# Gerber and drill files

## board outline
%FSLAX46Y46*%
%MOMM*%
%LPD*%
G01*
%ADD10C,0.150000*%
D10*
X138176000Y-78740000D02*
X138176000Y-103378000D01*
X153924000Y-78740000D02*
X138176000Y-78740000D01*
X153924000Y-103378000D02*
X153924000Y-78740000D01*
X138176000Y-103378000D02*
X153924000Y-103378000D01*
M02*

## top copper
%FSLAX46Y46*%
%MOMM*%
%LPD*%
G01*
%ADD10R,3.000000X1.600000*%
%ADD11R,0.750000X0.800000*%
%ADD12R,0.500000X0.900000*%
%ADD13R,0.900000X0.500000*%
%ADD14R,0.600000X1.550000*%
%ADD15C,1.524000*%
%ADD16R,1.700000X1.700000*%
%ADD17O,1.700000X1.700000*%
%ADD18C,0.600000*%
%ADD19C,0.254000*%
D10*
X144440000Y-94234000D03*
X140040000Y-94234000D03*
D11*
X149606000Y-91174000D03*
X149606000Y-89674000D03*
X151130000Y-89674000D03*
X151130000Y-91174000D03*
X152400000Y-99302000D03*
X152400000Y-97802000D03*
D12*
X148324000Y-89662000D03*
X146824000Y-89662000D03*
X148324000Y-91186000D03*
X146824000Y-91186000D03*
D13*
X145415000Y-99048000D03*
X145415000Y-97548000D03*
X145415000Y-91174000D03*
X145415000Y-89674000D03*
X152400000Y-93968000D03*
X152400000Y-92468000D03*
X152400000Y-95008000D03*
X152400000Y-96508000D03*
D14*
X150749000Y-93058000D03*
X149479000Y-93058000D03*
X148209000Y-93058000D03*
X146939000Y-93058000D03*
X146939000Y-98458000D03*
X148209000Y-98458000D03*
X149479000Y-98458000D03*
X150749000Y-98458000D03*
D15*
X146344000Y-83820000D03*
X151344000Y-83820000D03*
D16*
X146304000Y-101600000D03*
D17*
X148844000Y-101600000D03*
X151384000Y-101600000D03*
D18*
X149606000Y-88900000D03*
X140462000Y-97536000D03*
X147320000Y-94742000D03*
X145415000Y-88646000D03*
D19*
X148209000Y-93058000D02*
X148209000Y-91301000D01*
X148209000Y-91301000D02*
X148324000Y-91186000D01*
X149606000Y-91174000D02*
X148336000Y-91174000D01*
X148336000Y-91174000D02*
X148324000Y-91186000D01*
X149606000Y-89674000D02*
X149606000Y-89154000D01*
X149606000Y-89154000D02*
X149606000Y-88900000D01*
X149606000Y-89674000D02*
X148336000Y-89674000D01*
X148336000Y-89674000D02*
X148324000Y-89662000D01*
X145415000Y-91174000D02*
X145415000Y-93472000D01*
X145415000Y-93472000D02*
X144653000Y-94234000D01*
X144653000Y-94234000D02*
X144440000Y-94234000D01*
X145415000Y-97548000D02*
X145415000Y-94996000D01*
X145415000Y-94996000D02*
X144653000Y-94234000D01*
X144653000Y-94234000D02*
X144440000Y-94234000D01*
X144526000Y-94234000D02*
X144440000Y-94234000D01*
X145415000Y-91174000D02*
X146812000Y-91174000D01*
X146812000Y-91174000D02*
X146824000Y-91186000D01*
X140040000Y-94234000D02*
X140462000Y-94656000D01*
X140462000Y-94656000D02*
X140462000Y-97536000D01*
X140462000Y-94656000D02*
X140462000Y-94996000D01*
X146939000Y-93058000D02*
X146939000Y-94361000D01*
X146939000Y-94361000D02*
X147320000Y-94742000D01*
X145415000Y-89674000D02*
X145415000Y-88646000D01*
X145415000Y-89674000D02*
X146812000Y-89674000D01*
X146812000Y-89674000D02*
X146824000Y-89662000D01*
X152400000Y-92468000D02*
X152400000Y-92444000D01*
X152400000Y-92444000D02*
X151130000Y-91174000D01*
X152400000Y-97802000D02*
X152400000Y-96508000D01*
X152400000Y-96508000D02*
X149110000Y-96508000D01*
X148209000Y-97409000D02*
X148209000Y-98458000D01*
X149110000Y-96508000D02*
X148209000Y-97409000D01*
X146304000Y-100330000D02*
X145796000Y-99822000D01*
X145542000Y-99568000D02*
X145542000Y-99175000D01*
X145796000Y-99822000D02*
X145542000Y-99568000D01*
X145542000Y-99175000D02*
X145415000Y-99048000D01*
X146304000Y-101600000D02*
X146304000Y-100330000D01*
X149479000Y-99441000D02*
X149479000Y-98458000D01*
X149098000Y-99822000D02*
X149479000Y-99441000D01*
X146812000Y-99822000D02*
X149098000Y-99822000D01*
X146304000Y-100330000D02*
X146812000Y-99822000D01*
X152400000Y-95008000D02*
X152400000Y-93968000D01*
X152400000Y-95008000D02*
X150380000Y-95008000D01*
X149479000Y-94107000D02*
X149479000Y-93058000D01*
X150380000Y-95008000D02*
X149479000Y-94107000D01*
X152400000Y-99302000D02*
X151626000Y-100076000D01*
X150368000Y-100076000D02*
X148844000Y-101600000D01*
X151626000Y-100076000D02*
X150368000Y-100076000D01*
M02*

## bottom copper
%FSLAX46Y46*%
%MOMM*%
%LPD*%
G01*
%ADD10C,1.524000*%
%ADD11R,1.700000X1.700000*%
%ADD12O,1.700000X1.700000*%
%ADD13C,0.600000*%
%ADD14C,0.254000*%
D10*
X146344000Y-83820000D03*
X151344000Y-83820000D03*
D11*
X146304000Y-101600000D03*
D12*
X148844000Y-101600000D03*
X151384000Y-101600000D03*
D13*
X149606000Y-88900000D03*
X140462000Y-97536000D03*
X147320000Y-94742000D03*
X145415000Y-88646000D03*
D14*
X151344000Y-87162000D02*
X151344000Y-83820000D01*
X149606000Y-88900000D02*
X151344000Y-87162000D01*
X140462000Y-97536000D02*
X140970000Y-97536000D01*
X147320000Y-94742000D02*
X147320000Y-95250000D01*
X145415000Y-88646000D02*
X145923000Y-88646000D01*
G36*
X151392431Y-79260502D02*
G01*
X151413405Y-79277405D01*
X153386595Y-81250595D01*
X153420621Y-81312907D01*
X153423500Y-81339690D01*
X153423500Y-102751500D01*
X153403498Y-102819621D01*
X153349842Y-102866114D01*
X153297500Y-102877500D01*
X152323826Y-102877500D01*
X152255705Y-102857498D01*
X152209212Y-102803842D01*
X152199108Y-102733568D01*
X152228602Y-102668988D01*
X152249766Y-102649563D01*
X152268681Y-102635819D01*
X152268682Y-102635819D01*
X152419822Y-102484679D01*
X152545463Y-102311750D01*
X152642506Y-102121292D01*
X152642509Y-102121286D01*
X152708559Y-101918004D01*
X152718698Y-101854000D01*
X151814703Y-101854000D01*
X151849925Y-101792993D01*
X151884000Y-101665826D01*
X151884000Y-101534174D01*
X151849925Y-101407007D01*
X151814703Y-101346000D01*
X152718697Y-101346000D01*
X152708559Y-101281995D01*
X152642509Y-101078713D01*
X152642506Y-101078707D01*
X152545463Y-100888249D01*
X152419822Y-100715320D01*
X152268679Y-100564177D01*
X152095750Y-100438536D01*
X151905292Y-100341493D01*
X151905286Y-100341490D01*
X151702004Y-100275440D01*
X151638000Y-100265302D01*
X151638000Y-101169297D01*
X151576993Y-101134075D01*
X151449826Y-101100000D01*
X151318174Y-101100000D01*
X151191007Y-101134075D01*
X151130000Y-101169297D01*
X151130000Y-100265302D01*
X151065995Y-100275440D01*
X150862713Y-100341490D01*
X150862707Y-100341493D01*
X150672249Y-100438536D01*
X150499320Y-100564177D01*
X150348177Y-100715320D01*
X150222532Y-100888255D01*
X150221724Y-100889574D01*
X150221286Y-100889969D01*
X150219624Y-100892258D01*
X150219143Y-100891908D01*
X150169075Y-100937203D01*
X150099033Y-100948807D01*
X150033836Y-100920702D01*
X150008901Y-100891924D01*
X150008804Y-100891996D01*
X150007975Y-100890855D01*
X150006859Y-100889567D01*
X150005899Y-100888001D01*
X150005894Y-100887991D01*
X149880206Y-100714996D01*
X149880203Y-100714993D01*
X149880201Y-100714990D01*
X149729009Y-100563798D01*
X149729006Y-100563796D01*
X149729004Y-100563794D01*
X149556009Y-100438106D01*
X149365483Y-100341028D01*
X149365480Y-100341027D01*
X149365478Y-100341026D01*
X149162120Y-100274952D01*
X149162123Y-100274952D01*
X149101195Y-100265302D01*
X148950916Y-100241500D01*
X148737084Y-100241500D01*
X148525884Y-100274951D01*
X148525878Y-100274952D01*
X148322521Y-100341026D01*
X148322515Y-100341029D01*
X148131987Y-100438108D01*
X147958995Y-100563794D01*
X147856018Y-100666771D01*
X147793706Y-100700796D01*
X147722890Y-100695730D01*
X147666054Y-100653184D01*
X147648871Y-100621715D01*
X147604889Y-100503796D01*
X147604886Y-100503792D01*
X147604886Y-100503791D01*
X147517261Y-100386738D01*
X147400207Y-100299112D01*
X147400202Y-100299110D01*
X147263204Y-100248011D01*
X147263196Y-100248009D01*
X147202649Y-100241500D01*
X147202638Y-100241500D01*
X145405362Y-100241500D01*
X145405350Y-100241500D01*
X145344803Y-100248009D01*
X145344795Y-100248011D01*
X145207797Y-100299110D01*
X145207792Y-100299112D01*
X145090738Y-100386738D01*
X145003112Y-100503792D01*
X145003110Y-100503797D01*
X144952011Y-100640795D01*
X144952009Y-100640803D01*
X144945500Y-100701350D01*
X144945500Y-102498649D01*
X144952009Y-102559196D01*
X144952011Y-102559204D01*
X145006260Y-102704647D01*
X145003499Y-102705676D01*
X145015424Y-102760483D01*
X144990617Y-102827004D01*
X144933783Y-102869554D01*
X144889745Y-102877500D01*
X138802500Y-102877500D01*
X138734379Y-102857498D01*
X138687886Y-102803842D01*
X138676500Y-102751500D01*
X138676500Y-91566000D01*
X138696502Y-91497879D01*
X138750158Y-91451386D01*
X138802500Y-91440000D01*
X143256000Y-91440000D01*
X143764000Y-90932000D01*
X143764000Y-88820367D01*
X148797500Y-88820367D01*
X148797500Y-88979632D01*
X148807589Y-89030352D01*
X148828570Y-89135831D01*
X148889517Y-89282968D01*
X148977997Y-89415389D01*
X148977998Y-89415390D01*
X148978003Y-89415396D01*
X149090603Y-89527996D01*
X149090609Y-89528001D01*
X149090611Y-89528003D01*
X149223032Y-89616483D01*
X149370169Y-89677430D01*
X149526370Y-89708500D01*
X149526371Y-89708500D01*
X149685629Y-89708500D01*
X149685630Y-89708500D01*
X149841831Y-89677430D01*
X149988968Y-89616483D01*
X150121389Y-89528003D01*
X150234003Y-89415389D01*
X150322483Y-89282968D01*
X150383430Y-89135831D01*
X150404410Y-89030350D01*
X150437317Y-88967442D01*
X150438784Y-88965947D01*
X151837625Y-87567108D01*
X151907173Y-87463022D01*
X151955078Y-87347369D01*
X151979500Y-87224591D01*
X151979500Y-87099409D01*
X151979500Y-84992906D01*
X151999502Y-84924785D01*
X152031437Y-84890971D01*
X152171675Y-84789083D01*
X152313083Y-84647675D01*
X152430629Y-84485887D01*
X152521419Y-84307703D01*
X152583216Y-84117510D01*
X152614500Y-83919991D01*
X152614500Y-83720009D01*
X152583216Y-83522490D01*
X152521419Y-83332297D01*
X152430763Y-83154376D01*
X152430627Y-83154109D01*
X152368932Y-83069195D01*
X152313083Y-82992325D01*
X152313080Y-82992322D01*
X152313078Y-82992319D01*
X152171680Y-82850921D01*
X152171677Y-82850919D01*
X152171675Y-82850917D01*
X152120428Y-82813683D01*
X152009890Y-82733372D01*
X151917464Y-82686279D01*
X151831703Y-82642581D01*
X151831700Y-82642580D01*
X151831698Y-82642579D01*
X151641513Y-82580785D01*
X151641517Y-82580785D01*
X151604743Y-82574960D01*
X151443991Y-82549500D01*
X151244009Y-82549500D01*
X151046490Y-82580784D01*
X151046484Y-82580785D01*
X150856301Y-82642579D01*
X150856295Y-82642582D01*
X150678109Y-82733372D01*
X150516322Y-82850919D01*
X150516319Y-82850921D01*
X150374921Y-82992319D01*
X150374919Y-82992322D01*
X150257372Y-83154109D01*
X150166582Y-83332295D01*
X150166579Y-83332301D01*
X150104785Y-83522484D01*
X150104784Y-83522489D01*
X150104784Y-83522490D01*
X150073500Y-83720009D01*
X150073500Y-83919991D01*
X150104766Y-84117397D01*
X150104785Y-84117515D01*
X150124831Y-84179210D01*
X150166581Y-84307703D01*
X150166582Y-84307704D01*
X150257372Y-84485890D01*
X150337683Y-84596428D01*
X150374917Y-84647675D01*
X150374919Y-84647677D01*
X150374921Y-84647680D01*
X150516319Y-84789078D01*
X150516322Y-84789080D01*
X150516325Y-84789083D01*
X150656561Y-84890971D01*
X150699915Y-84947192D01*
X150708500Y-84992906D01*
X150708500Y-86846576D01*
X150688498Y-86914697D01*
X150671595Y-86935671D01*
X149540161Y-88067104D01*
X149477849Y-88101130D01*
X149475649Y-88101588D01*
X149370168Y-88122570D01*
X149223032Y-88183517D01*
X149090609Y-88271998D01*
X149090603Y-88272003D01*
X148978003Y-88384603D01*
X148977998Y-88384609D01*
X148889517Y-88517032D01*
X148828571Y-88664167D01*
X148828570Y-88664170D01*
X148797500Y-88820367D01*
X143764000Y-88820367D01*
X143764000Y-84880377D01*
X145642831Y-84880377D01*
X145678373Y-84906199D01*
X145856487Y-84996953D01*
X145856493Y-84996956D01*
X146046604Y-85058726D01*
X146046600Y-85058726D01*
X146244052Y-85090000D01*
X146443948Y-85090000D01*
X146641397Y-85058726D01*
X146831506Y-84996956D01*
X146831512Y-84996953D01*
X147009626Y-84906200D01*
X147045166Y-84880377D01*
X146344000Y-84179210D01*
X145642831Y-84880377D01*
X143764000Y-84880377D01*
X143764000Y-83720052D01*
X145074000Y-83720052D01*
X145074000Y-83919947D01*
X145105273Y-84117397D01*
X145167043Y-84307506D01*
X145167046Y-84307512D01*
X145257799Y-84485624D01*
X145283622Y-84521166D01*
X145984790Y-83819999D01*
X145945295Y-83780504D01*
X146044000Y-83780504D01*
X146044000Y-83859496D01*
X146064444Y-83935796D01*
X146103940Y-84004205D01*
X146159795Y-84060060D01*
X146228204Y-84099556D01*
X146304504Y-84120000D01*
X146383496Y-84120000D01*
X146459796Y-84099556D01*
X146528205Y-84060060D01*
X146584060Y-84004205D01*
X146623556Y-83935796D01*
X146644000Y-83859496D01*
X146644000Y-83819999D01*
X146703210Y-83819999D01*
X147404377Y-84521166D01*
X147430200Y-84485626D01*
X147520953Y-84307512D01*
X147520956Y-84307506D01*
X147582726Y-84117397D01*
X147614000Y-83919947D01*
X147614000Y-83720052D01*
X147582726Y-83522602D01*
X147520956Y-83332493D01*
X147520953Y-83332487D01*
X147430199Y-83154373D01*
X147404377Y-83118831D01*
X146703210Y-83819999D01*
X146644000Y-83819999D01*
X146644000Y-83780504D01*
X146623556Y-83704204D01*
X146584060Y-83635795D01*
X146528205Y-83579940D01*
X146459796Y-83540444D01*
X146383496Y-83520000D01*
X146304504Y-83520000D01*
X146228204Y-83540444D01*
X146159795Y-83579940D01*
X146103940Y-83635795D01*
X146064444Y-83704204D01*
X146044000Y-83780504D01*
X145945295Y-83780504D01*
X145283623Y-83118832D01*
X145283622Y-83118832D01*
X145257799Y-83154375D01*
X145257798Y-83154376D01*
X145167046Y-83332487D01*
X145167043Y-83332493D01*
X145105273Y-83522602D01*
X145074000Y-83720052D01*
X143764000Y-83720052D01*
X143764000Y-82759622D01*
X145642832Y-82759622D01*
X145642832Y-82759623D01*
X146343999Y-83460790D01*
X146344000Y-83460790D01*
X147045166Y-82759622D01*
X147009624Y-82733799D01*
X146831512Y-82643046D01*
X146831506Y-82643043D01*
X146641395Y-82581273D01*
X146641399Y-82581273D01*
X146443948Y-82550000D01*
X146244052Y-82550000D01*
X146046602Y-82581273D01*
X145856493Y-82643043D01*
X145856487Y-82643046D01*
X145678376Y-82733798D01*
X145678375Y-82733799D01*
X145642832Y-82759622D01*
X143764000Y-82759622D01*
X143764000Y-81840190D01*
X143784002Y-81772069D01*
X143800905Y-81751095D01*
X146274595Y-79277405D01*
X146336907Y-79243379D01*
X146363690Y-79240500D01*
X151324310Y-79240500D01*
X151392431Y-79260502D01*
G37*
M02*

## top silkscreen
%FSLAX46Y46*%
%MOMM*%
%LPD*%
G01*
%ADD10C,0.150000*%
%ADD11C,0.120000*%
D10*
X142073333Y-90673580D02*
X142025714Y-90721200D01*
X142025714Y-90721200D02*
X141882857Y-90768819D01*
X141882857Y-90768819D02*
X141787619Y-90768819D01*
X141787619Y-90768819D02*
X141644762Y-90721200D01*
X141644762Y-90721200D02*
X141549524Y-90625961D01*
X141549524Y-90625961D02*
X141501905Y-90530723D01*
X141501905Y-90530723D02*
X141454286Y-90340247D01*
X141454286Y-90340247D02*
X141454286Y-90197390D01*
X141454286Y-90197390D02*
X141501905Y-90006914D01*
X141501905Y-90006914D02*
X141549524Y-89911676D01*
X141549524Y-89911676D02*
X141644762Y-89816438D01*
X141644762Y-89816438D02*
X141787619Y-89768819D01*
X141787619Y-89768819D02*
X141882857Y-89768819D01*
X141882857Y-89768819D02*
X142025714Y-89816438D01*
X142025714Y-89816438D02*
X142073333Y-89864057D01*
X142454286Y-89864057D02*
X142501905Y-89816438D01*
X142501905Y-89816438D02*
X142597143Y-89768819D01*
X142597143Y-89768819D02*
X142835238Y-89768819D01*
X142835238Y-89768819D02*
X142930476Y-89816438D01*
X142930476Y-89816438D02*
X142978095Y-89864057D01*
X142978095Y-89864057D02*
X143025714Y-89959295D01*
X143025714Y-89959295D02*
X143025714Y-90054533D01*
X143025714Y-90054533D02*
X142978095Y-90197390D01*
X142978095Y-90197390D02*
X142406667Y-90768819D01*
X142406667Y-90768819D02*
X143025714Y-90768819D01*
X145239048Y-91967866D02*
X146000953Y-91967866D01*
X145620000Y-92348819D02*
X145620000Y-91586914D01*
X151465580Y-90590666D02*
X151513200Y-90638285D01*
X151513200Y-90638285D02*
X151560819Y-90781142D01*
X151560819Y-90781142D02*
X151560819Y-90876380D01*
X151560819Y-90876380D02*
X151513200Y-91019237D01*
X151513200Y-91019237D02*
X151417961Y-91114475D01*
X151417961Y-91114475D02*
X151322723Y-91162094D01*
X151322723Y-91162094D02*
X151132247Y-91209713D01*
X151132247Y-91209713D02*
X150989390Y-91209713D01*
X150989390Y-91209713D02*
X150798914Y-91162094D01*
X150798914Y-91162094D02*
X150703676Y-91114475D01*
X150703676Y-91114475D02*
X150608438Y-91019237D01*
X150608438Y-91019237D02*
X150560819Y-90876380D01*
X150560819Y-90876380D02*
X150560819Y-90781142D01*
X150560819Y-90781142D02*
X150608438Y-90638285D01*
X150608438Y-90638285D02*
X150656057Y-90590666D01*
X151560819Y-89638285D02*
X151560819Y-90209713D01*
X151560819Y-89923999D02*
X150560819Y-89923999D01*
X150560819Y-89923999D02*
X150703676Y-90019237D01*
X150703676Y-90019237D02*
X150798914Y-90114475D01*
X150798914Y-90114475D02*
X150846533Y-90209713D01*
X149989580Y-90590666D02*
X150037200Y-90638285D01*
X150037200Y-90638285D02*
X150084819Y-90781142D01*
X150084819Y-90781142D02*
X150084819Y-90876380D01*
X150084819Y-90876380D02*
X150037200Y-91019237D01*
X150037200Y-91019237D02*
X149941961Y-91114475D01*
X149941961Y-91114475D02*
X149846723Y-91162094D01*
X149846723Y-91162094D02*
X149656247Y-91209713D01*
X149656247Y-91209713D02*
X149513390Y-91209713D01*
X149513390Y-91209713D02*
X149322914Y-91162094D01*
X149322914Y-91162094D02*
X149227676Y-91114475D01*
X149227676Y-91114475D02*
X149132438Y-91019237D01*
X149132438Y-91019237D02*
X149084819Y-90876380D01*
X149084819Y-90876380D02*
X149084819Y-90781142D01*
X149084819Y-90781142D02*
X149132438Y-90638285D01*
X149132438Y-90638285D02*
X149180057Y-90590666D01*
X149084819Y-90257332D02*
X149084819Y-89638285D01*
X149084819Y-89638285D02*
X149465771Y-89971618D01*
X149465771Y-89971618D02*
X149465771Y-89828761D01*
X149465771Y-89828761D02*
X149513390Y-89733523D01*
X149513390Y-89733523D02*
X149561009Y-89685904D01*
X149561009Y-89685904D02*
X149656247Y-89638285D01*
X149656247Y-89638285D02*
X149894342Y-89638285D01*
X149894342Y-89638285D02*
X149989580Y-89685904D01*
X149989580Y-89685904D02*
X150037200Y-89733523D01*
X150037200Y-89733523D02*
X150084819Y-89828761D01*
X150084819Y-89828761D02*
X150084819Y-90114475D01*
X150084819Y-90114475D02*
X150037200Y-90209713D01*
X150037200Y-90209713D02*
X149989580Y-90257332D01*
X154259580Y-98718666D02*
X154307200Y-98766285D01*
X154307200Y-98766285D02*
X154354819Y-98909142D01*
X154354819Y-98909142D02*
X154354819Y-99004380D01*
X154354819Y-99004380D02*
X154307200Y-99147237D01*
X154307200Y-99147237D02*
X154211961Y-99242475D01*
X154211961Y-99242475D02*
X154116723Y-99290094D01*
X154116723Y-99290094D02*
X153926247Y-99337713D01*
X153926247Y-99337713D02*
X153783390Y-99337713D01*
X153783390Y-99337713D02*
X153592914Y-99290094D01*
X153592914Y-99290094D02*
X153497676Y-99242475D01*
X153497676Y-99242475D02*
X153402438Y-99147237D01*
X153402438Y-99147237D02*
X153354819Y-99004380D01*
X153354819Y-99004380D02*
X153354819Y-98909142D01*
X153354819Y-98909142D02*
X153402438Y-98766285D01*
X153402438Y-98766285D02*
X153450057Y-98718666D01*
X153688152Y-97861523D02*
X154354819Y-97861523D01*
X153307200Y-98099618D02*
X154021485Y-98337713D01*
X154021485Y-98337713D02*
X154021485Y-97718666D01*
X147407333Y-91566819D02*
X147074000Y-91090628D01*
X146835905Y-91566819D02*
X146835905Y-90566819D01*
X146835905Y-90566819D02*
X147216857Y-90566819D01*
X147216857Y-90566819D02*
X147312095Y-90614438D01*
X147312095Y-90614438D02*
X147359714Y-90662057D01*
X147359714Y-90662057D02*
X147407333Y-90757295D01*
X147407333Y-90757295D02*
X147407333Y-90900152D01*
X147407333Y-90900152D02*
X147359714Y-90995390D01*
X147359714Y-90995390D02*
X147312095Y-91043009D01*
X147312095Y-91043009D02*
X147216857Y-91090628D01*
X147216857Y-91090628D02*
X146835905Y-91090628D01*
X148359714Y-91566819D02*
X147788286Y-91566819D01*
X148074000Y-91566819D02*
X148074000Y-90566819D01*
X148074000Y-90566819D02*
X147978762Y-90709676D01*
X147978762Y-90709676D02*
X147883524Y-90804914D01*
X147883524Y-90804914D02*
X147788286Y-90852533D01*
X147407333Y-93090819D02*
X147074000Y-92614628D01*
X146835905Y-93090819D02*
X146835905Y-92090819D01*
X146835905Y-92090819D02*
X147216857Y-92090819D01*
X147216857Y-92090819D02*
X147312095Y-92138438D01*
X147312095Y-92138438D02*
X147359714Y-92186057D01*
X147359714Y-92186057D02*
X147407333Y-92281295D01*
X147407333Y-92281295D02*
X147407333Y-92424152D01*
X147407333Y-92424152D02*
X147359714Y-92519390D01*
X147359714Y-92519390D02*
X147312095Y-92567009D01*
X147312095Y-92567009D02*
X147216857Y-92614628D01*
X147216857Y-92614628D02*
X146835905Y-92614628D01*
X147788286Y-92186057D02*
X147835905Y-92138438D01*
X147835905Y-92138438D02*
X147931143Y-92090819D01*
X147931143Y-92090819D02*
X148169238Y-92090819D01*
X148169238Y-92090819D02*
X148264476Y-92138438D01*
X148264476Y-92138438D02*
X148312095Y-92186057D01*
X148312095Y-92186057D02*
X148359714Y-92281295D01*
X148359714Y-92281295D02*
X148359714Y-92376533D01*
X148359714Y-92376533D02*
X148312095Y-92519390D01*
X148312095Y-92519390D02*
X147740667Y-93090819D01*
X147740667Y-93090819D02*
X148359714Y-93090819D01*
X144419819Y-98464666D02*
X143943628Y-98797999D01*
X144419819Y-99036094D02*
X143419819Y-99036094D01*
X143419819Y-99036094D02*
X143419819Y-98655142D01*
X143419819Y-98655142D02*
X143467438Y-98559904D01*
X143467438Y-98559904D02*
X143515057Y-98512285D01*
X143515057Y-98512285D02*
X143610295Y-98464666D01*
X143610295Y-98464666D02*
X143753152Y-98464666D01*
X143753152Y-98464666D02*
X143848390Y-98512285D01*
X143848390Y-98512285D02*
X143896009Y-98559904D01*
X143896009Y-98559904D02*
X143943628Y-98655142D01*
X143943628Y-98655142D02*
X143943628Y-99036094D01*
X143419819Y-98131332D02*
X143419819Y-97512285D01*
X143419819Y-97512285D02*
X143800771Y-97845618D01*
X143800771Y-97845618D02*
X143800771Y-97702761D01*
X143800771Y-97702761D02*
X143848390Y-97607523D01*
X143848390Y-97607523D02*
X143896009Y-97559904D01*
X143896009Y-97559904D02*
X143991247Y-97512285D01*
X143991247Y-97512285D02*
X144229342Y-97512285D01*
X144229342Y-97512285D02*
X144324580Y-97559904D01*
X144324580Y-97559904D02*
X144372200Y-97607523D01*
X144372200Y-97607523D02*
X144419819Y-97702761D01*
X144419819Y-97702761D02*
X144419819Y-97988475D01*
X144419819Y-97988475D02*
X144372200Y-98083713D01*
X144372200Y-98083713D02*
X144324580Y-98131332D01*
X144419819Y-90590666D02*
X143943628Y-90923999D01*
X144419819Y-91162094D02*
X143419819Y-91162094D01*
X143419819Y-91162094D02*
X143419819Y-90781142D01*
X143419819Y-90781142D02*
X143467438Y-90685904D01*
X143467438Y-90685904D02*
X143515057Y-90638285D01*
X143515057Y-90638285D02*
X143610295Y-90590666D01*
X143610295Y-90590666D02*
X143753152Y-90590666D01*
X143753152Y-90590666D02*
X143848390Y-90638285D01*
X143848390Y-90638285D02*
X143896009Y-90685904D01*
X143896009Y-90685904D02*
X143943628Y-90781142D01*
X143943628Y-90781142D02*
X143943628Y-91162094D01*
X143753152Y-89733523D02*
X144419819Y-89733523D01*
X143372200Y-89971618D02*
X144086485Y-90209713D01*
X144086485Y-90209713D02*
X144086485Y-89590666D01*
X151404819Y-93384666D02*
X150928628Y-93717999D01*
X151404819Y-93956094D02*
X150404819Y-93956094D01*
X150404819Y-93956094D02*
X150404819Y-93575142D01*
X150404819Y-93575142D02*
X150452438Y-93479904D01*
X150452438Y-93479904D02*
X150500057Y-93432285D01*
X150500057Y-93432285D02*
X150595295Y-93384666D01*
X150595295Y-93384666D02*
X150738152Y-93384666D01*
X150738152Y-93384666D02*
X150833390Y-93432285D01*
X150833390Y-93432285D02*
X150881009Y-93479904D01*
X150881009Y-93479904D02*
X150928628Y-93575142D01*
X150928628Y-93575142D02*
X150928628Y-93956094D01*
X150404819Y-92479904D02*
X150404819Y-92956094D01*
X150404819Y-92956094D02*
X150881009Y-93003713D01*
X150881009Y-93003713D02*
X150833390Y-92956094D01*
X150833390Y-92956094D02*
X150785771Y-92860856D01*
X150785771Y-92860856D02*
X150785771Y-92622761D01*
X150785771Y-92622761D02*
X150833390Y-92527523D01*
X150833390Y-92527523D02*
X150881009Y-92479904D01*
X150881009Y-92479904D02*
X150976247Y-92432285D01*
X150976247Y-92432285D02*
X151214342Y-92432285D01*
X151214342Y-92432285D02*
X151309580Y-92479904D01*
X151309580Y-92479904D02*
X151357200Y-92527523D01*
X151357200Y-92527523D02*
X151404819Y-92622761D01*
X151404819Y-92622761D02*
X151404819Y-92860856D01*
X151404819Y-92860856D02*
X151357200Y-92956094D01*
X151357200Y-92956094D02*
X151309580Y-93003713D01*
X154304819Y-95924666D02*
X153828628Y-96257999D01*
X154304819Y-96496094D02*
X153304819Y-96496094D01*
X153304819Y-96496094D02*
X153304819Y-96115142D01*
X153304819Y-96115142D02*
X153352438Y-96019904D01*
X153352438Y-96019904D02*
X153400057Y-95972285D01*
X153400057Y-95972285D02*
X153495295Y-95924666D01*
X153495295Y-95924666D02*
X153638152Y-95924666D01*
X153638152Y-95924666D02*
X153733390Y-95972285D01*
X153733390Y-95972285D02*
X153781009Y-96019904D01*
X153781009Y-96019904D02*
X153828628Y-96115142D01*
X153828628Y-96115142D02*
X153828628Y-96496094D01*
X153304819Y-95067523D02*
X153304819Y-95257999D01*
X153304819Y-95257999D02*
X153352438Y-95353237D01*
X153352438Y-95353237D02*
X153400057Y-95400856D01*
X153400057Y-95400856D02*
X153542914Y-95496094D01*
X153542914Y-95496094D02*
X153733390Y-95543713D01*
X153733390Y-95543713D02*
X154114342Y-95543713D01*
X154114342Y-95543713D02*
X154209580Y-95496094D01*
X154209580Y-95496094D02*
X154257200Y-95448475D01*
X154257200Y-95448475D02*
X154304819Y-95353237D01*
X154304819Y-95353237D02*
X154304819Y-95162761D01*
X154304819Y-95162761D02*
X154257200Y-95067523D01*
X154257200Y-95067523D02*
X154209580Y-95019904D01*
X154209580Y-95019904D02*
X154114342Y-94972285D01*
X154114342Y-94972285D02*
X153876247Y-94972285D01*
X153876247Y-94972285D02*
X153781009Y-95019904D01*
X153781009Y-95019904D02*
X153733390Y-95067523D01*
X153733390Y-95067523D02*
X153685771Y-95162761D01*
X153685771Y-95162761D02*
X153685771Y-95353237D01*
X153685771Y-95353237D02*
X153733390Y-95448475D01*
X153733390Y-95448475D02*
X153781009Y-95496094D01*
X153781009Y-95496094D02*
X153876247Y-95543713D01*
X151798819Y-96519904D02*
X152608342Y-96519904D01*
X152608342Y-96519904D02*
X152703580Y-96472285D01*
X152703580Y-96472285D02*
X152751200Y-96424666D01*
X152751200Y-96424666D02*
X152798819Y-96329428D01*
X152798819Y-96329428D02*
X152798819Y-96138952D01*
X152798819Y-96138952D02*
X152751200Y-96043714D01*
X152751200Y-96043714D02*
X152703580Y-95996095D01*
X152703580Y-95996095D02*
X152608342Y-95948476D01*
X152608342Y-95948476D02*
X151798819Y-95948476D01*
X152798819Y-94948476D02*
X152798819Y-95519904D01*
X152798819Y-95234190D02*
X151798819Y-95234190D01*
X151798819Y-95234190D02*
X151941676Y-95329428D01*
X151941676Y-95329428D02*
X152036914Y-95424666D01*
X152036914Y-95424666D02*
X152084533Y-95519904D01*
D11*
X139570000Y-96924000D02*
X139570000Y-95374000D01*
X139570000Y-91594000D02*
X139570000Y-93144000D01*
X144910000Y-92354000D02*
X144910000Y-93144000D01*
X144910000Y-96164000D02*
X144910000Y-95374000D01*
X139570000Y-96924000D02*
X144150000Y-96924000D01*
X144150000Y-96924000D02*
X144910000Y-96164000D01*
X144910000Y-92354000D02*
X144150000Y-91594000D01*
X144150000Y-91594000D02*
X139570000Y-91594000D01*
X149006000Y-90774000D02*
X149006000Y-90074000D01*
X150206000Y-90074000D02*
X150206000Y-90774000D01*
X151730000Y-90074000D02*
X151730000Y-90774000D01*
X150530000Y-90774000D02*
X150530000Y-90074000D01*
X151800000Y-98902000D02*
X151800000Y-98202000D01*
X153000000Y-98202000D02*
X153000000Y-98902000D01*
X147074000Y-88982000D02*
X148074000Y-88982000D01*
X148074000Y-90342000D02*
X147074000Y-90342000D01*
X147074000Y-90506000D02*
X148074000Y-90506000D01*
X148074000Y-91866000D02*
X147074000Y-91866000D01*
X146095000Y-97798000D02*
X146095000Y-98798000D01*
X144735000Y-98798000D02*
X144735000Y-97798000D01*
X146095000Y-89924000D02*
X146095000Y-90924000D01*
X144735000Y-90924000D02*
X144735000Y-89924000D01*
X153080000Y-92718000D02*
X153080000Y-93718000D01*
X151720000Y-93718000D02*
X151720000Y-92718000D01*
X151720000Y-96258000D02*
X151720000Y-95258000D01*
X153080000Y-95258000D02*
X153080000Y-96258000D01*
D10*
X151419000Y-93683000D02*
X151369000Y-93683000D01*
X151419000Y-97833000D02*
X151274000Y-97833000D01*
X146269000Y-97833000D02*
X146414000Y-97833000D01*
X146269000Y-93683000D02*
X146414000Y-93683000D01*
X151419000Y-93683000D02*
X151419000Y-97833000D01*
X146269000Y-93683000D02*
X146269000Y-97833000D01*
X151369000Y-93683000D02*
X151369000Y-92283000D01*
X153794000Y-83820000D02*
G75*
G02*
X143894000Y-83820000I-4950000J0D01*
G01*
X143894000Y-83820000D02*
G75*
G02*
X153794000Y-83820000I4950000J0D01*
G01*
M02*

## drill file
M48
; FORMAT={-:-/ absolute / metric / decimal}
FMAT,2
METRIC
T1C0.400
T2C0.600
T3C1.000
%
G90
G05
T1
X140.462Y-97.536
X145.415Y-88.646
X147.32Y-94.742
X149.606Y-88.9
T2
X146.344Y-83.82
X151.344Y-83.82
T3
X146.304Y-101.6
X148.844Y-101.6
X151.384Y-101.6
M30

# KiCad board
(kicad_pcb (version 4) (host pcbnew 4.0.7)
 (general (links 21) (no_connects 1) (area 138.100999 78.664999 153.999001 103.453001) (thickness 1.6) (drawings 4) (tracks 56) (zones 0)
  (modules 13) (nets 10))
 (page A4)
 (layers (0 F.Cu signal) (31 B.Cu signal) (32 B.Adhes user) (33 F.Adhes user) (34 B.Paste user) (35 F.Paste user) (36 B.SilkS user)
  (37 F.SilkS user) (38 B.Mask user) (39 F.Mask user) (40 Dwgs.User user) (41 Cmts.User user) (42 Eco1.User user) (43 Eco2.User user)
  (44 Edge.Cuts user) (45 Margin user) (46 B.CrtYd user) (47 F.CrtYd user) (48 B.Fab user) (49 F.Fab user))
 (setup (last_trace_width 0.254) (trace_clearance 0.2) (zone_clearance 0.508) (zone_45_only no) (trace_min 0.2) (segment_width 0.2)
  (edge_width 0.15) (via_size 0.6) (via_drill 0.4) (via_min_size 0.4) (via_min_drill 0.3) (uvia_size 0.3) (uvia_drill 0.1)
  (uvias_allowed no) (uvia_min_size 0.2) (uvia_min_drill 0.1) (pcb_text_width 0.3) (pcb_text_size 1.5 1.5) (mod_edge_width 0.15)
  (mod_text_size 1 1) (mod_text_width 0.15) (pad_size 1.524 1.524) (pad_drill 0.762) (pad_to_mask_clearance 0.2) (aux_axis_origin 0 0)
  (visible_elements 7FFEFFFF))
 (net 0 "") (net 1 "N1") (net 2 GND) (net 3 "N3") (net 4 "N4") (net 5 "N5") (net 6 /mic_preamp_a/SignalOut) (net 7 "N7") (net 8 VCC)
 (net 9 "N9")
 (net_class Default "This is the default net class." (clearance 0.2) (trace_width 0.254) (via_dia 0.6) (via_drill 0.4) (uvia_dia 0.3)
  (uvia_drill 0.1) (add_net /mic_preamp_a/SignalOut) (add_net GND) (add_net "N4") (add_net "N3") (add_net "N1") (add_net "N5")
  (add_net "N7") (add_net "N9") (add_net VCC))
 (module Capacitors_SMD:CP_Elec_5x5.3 (layer F.Cu) (at 142.24 94.234 180)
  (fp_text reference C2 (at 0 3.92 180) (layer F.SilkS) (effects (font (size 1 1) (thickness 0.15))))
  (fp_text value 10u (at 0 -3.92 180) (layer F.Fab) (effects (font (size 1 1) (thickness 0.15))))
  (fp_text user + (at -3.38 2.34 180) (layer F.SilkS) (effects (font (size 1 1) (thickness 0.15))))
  (fp_line (start 2.67 -2.69) (end 2.67 -1.14) (layer F.SilkS) (width 0.12))
  (fp_line (start 2.67 2.64) (end 2.67 1.09) (layer F.SilkS) (width 0.12))
  (fp_line (start -2.67 1.88) (end -2.67 1.09) (layer F.SilkS) (width 0.12))
  (fp_line (start -2.67 -1.93) (end -2.67 -1.14) (layer F.SilkS) (width 0.12))
  (fp_line (start 2.67 -2.69) (end -1.91 -2.69) (layer F.SilkS) (width 0.12))
  (fp_line (start -1.91 -2.69) (end -2.67 -1.93) (layer F.SilkS) (width 0.12))
  (fp_line (start -2.67 1.88) (end -1.91 2.64) (layer F.SilkS) (width 0.12))
  (fp_line (start -1.91 2.64) (end 2.67 2.64) (layer F.SilkS) (width 0.12))
  (pad 1 smd rect (at -2.2 0) (size 3 1.6) (layers F.Cu F.Paste F.Mask) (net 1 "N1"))
  (pad 2 smd rect (at 2.2 0) (size 3 1.6) (layers F.Cu F.Paste F.Mask) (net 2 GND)))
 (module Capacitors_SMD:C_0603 (layer F.Cu) (at 149.606 90.424 270)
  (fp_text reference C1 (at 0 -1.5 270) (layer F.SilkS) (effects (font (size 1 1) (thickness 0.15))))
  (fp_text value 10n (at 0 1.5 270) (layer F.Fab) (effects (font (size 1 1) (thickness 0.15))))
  (fp_line (start 0.35 0.6) (end -0.35 0.6) (layer F.SilkS) (width 0.12))
  (fp_line (start -0.35 -0.6) (end 0.35 -0.6) (layer F.SilkS) (width 0.12))
  (pad 2 smd rect (at 0.75 0 270) (size 0.8 0.75) (layers F.Cu F.Paste F.Mask) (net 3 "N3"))
  (pad 1 smd rect (at -0.75 0 270) (size 0.8 0.75) (layers F.Cu F.Paste F.Mask) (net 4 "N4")))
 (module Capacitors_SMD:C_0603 (layer F.Cu) (at 151.13 90.424 90)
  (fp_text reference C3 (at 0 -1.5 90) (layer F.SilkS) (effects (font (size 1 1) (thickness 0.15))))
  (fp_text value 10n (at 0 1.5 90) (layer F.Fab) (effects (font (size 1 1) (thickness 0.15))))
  (fp_line (start 0.35 0.6) (end -0.35 0.6) (layer F.SilkS) (width 0.12))
  (fp_line (start -0.35 -0.6) (end 0.35 -0.6) (layer F.SilkS) (width 0.12))
  (pad 2 smd rect (at 0.75 0 90) (size 0.8 0.75) (layers F.Cu F.Paste F.Mask) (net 2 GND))
  (pad 1 smd rect (at -0.75 0 90) (size 0.8 0.75) (layers F.Cu F.Paste F.Mask) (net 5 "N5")))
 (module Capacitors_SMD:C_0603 (layer F.Cu) (at 152.4 98.552 270)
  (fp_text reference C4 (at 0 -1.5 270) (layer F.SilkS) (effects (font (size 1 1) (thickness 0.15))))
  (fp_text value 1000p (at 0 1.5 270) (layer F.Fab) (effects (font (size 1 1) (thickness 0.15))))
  (fp_line (start 0.35 0.6) (end -0.35 0.6) (layer F.SilkS) (width 0.12))
  (fp_line (start -0.35 -0.6) (end 0.35 -0.6) (layer F.SilkS) (width 0.12))
  (pad 2 smd rect (at 0.75 0 270) (size 0.8 0.75) (layers F.Cu F.Paste F.Mask) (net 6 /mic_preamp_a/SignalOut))
  (pad 1 smd rect (at -0.75 0 270) (size 0.8 0.75) (layers F.Cu F.Paste F.Mask) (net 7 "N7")))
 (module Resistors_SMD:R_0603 (layer F.Cu) (at 147.574 89.662 180)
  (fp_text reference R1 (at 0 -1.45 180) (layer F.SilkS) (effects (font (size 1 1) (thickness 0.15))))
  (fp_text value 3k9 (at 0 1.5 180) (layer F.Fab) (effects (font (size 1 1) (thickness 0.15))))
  (fp_line (start 0.5 0.68) (end -0.5 0.68) (layer F.SilkS) (width 0.12))
  (fp_line (start -0.5 -0.68) (end 0.5 -0.68) (layer F.SilkS) (width 0.12))
  (pad 1 smd rect (at -0.75 0 180) (size 0.5 0.9) (layers F.Cu F.Paste F.Mask) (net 4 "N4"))
  (pad 2 smd rect (at 0.75 0 180) (size 0.5 0.9) (layers F.Cu F.Paste F.Mask) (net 2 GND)))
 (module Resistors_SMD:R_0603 (layer F.Cu) (at 147.574 91.186 180)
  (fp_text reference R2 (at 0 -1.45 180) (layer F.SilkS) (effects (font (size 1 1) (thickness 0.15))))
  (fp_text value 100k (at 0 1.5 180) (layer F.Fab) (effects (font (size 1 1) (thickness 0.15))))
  (fp_line (start 0.5 0.68) (end -0.5 0.68) (layer F.SilkS) (width 0.12))
  (fp_line (start -0.5 -0.68) (end 0.5 -0.68) (layer F.SilkS) (width 0.12))
  (pad 1 smd rect (at -0.75 0 180) (size 0.5 0.9) (layers F.Cu F.Paste F.Mask) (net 3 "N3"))
  (pad 2 smd rect (at 0.75 0 180) (size 0.5 0.9) (layers F.Cu F.Paste F.Mask) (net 1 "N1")))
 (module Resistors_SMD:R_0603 (layer F.Cu) (at 145.415 98.298 90)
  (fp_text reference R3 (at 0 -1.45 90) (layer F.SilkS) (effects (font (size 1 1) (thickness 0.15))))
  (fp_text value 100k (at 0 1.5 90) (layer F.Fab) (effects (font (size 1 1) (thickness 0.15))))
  (fp_line (start 0.5 0.68) (end -0.5 0.68) (layer F.SilkS) (width 0.12))
  (fp_line (start -0.5 -0.68) (end 0.5 -0.68) (layer F.SilkS) (width 0.12))
  (pad 1 smd rect (at -0.75 0 90) (size 0.5 0.9) (layers F.Cu F.Paste F.Mask) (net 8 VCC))
  (pad 2 smd rect (at 0.75 0 90) (size 0.5 0.9) (layers F.Cu F.Paste F.Mask) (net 1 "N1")))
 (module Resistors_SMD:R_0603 (layer F.Cu) (at 145.415 90.424 90)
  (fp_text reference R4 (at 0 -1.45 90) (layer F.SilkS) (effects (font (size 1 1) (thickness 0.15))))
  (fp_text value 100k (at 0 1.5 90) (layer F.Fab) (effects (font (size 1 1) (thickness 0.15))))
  (fp_line (start 0.5 0.68) (end -0.5 0.68) (layer F.SilkS) (width 0.12))
  (fp_line (start -0.5 -0.68) (end 0.5 -0.68) (layer F.SilkS) (width 0.12))
  (pad 1 smd rect (at -0.75 0 90) (size 0.5 0.9) (layers F.Cu F.Paste F.Mask) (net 1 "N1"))
  (pad 2 smd rect (at 0.75 0 90) (size 0.5 0.9) (layers F.Cu F.Paste F.Mask) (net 2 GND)))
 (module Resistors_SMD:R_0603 (layer F.Cu) (at 152.4 93.218 90)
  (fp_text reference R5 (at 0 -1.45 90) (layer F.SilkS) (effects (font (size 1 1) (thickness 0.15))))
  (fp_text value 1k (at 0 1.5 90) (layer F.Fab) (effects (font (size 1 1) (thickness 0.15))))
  (fp_line (start 0.5 0.68) (end -0.5 0.68) (layer F.SilkS) (width 0.12))
  (fp_line (start -0.5 -0.68) (end 0.5 -0.68) (layer F.SilkS) (width 0.12))
  (pad 1 smd rect (at -0.75 0 90) (size 0.5 0.9) (layers F.Cu F.Paste F.Mask) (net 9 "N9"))
  (pad 2 smd rect (at 0.75 0 90) (size 0.5 0.9) (layers F.Cu F.Paste F.Mask) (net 5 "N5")))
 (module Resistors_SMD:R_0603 (layer F.Cu) (at 152.4 95.758 270)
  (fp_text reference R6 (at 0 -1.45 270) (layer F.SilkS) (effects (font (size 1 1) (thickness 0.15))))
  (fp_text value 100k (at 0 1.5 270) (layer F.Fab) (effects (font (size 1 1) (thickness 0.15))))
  (fp_line (start 0.5 0.68) (end -0.5 0.68) (layer F.SilkS) (width 0.12))
  (fp_line (start -0.5 -0.68) (end 0.5 -0.68) (layer F.SilkS) (width 0.12))
  (pad 1 smd rect (at -0.75 0 270) (size 0.5 0.9) (layers F.Cu F.Paste F.Mask) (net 9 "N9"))
  (pad 2 smd rect (at 0.75 0 270) (size 0.5 0.9) (layers F.Cu F.Paste F.Mask) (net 7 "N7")))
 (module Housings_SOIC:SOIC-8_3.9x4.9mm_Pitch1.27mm (layer F.Cu) (at 148.844 95.758 270)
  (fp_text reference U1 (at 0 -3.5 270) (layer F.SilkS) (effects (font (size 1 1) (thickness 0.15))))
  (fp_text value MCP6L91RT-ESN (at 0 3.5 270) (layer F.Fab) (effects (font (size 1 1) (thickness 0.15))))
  (fp_line (start -2.075 -2.575) (end -2.075 -2.525) (layer F.SilkS) (width 0.15))
  (fp_line (start 2.075 -2.575) (end 2.075 -2.43) (layer F.SilkS) (width 0.15))
  (fp_line (start 2.075 2.575) (end 2.075 2.43) (layer F.SilkS) (width 0.15))
  (fp_line (start -2.075 2.575) (end -2.075 2.43) (layer F.SilkS) (width 0.15))
  (fp_line (start -2.075 -2.575) (end 2.075 -2.575) (layer F.SilkS) (width 0.15))
  (fp_line (start -2.075 2.575) (end 2.075 2.575) (layer F.SilkS) (width 0.15))
  (fp_line (start -2.075 -2.525) (end -3.475 -2.525) (layer F.SilkS) (width 0.15))
  (pad 1 smd rect (at -2.7 -1.905 270) (size 1.55 0.6) (layers F.Cu F.Paste F.Mask))
  (pad 2 smd rect (at -2.7 -0.635 270) (size 1.55 0.6) (layers F.Cu F.Paste F.Mask) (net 9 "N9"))
  (pad 3 smd rect (at -2.7 0.635 270) (size 1.55 0.6) (layers F.Cu F.Paste F.Mask) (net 3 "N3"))
  (pad 4 smd rect (at -2.7 1.905 270) (size 1.55 0.6) (layers F.Cu F.Paste F.Mask) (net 2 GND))
  (pad 5 smd rect (at 2.7 1.905 270) (size 1.55 0.6) (layers F.Cu F.Paste F.Mask))
  (pad 6 smd rect (at 2.7 0.635 270) (size 1.55 0.6) (layers F.Cu F.Paste F.Mask) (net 7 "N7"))
  (pad 7 smd rect (at 2.7 -0.635 270) (size 1.55 0.6) (layers F.Cu F.Paste F.Mask) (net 8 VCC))
  (pad 8 smd rect (at 2.7 -1.905 270) (size 1.55 0.6) (layers F.Cu F.Paste F.Mask)))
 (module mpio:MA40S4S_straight (layer F.Cu) (at 148.844 83.82)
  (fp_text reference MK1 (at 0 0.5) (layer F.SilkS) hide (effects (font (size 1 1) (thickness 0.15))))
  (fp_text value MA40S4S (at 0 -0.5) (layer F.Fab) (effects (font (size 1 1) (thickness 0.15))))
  (fp_circle (center 0 0) (end 4.95 0) (layer F.SilkS) (width 0.15))
  (pad 1 thru_hole circle (at -2.5 0) (size 1.524 1.524) (drill 0.6) (layers *.Cu *.Mask) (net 2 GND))
  (pad 2 thru_hole circle (at 2.5 0) (size 1.524 1.524) (drill 0.6) (layers *.Cu *.Mask) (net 4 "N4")))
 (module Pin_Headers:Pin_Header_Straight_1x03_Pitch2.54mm (layer B.Cu) (at 146.304 101.6 270)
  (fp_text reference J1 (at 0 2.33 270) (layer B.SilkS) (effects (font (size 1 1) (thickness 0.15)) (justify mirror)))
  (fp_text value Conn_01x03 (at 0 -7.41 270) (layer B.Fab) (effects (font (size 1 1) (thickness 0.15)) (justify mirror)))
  (pad 1 thru_hole rect (at 0 0 270) (size 1.7 1.7) (drill 1) (layers *.Cu *.Mask) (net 8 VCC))
  (pad 2 thru_hole oval (at 0 -2.54 270) (size 1.7 1.7) (drill 1) (layers *.Cu *.Mask) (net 6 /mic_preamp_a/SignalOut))
  (pad 3 thru_hole oval (at 0 -5.08 270) (size 1.7 1.7) (drill 1) (layers *.Cu *.Mask) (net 2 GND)))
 (gr_line (start 138.176 78.74) (end 138.176 103.378) (angle 90) (layer Edge.Cuts) (width 0.15))
 (gr_line (start 153.924 78.74) (end 138.176 78.74) (angle 90) (layer Edge.Cuts) (width 0.15))
 (gr_line (start 153.924 103.378) (end 153.924 78.74) (angle 90) (layer Edge.Cuts) (width 0.15))
 (gr_line (start 138.176 103.378) (end 153.924 103.378) (angle 90) (layer Edge.Cuts) (width 0.15))
 (segment (start 148.209 93.058) (end 148.209 91.301) (width 0.254) (layer F.Cu) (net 3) (status 10))
 (segment (start 148.209 91.301) (end 148.324 91.186) (width 0.254) (layer F.Cu) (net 3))
 (segment (start 149.606 91.174) (end 148.336 91.174) (width 0.254) (layer F.Cu) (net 3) (status 20))
 (segment (start 148.336 91.174) (end 148.324 91.186) (width 0.254) (layer F.Cu) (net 3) (status 30))
 (segment (start 149.606 89.674) (end 149.606 89.154) (width 0.254) (layer F.Cu) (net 4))
 (segment (start 151.344 87.162) (end 151.344 83.82) (width 0.254) (layer B.Cu) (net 4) (status 20))
 (segment (start 149.606 88.9) (end 151.344 87.162) (width 0.254) (layer B.Cu) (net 4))
 (via (at 149.606 88.9) (size 0.6) (drill 0.4) (layers F.Cu B.Cu) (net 4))
 (segment (start 149.606 89.154) (end 149.606 88.9) (width 0.254) (layer F.Cu) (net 4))
 (segment (start 149.606 89.674) (end 148.336 89.674) (width 0.254) (layer F.Cu) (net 4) (status 10))
 (segment (start 148.336 89.674) (end 148.324 89.662) (width 0.254) (layer F.Cu) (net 4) (status 30))
 (segment (start 145.415 91.174) (end 145.415 93.472) (width 0.254) (layer F.Cu) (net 1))
 (segment (start 145.415 93.472) (end 144.653 94.234) (width 0.254) (layer F.Cu) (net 1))
 (segment (start 144.653 94.234) (end 144.44 94.234) (width 0.254) (layer F.Cu) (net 1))
 (segment (start 145.415 97.548) (end 145.415 94.996) (width 0.254) (layer F.Cu) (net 1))
 (segment (start 145.415 94.996) (end 144.653 94.234) (width 0.254) (layer F.Cu) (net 1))
 (segment (start 144.653 94.234) (end 144.44 94.234) (width 0.254) (layer F.Cu) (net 1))
 (segment (start 144.526 94.234) (end 144.44 94.234) (width 0.254) (layer F.Cu) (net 1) (status 30))
 (segment (start 145.415 91.174) (end 146.812 91.174) (width 0.254) (layer F.Cu) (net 1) (status 10))
 (segment (start 146.812 91.174) (end 146.824 91.186) (width 0.254) (layer F.Cu) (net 1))
 (segment (start 140.04 94.234) (end 140.462 94.656) (width 0.254) (layer F.Cu) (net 2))
 (segment (start 140.462 94.656) (end 140.462 97.536) (width 0.254) (layer F.Cu) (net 2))
 (segment (start 140.462 97.536) (end 140.97 97.536) (width 0.254) (layer B.Cu) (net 2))
 (via (at 140.462 97.536) (size 0.6) (drill 0.4) (layers F.Cu B.Cu) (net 2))
 (segment (start 140.462 94.656) (end 140.462 94.996) (width 0.254) (layer F.Cu) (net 2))
 (segment (start 146.939 93.058) (end 146.939 94.361) (width 0.254) (layer F.Cu) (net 2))
 (segment (start 147.32 94.742) (end 147.32 95.25) (width 0.254) (layer B.Cu) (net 2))
 (via (at 147.32 94.742) (size 0.6) (drill 0.4) (layers F.Cu B.Cu) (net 2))
 (segment (start 146.939 94.361) (end 147.32 94.742) (width 0.254) (layer F.Cu) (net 2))
 (segment (start 145.415 89.674) (end 145.415 88.646) (width 0.254) (layer F.Cu) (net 2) (status 10))
 (segment (start 145.415 88.646) (end 145.923 88.646) (width 0.254) (layer B.Cu) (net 2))
 (via (at 145.415 88.646) (size 0.6) (drill 0.4) (layers F.Cu B.Cu) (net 2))
 (segment (start 145.415 89.674) (end 146.812 89.674) (width 0.254) (layer F.Cu) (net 2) (status 10))
 (segment (start 146.812 89.674) (end 146.824 89.662) (width 0.254) (layer F.Cu) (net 2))
 (segment (start 152.4 92.468) (end 152.4 92.444) (width 0.254) (layer F.Cu) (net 5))
 (segment (start 152.4 92.444) (end 151.13 91.174) (width 0.254) (layer F.Cu) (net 5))
 (segment (start 152.4 97.802) (end 152.4 96.508) (width 0.254) (layer F.Cu) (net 7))
 (segment (start 152.4 96.508) (end 149.11 96.508) (width 0.254) (layer F.Cu) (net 7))
 (segment (start 148.209 97.409) (end 148.209 98.458) (width 0.254) (layer F.Cu) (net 7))
 (segment (start 149.11 96.508) (end 148.209 97.409) (width 0.254) (layer F.Cu) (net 7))
 (segment (start 146.304 100.33) (end 145.796 99.822) (width 0.254) (layer F.Cu) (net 8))
 (segment (start 145.542 99.568) (end 145.542 99.175) (width 0.254) (layer F.Cu) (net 8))
 (segment (start 145.796 99.822) (end 145.542 99.568) (width 0.254) (layer F.Cu) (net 8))
 (segment (start 145.542 99.175) (end 145.415 99.048) (width 0.254) (layer F.Cu) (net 8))
 (segment (start 146.304 101.6) (end 146.304 100.33) (width 0.254) (layer F.Cu) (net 8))
 (segment (start 149.479 99.441) (end 149.479 98.458) (width 0.254) (layer F.Cu) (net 8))
 (segment (start 149.098 99.822) (end 149.479 99.441) (width 0.254) (layer F.Cu) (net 8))
 (segment (start 146.812 99.822) (end 149.098 99.822) (width 0.254) (layer F.Cu) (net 8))
 (segment (start 146.304 100.33) (end 146.812 99.822) (width 0.254) (layer F.Cu) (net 8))
 (segment (start 152.4 95.008) (end 152.4 93.968) (width 0.254) (layer F.Cu) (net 9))
 (segment (start 152.4 95.008) (end 150.38 95.008) (width 0.254) (layer F.Cu) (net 9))
 (segment (start 149.479 94.107) (end 149.479 93.058) (width 0.254) (layer F.Cu) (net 9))
 (segment (start 150.38 95.008) (end 149.479 94.107) (width 0.254) (layer F.Cu) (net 9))
 (segment (start 152.4 99.302) (end 151.626 100.076) (width 0.254) (layer F.Cu) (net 6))
 (segment (start 150.368 100.076) (end 148.844 101.6) (width 0.254) (layer F.Cu) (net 6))
 (segment (start 151.626 100.076) (end 150.368 100.076) (width 0.254) (layer F.Cu) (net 6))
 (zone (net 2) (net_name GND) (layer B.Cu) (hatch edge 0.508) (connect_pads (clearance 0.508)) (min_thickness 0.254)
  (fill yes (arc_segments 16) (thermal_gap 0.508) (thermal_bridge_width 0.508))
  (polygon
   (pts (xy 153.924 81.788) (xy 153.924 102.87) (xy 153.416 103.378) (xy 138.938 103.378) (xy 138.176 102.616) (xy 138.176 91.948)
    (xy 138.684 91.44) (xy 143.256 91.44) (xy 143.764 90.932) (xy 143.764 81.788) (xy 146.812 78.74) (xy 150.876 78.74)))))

